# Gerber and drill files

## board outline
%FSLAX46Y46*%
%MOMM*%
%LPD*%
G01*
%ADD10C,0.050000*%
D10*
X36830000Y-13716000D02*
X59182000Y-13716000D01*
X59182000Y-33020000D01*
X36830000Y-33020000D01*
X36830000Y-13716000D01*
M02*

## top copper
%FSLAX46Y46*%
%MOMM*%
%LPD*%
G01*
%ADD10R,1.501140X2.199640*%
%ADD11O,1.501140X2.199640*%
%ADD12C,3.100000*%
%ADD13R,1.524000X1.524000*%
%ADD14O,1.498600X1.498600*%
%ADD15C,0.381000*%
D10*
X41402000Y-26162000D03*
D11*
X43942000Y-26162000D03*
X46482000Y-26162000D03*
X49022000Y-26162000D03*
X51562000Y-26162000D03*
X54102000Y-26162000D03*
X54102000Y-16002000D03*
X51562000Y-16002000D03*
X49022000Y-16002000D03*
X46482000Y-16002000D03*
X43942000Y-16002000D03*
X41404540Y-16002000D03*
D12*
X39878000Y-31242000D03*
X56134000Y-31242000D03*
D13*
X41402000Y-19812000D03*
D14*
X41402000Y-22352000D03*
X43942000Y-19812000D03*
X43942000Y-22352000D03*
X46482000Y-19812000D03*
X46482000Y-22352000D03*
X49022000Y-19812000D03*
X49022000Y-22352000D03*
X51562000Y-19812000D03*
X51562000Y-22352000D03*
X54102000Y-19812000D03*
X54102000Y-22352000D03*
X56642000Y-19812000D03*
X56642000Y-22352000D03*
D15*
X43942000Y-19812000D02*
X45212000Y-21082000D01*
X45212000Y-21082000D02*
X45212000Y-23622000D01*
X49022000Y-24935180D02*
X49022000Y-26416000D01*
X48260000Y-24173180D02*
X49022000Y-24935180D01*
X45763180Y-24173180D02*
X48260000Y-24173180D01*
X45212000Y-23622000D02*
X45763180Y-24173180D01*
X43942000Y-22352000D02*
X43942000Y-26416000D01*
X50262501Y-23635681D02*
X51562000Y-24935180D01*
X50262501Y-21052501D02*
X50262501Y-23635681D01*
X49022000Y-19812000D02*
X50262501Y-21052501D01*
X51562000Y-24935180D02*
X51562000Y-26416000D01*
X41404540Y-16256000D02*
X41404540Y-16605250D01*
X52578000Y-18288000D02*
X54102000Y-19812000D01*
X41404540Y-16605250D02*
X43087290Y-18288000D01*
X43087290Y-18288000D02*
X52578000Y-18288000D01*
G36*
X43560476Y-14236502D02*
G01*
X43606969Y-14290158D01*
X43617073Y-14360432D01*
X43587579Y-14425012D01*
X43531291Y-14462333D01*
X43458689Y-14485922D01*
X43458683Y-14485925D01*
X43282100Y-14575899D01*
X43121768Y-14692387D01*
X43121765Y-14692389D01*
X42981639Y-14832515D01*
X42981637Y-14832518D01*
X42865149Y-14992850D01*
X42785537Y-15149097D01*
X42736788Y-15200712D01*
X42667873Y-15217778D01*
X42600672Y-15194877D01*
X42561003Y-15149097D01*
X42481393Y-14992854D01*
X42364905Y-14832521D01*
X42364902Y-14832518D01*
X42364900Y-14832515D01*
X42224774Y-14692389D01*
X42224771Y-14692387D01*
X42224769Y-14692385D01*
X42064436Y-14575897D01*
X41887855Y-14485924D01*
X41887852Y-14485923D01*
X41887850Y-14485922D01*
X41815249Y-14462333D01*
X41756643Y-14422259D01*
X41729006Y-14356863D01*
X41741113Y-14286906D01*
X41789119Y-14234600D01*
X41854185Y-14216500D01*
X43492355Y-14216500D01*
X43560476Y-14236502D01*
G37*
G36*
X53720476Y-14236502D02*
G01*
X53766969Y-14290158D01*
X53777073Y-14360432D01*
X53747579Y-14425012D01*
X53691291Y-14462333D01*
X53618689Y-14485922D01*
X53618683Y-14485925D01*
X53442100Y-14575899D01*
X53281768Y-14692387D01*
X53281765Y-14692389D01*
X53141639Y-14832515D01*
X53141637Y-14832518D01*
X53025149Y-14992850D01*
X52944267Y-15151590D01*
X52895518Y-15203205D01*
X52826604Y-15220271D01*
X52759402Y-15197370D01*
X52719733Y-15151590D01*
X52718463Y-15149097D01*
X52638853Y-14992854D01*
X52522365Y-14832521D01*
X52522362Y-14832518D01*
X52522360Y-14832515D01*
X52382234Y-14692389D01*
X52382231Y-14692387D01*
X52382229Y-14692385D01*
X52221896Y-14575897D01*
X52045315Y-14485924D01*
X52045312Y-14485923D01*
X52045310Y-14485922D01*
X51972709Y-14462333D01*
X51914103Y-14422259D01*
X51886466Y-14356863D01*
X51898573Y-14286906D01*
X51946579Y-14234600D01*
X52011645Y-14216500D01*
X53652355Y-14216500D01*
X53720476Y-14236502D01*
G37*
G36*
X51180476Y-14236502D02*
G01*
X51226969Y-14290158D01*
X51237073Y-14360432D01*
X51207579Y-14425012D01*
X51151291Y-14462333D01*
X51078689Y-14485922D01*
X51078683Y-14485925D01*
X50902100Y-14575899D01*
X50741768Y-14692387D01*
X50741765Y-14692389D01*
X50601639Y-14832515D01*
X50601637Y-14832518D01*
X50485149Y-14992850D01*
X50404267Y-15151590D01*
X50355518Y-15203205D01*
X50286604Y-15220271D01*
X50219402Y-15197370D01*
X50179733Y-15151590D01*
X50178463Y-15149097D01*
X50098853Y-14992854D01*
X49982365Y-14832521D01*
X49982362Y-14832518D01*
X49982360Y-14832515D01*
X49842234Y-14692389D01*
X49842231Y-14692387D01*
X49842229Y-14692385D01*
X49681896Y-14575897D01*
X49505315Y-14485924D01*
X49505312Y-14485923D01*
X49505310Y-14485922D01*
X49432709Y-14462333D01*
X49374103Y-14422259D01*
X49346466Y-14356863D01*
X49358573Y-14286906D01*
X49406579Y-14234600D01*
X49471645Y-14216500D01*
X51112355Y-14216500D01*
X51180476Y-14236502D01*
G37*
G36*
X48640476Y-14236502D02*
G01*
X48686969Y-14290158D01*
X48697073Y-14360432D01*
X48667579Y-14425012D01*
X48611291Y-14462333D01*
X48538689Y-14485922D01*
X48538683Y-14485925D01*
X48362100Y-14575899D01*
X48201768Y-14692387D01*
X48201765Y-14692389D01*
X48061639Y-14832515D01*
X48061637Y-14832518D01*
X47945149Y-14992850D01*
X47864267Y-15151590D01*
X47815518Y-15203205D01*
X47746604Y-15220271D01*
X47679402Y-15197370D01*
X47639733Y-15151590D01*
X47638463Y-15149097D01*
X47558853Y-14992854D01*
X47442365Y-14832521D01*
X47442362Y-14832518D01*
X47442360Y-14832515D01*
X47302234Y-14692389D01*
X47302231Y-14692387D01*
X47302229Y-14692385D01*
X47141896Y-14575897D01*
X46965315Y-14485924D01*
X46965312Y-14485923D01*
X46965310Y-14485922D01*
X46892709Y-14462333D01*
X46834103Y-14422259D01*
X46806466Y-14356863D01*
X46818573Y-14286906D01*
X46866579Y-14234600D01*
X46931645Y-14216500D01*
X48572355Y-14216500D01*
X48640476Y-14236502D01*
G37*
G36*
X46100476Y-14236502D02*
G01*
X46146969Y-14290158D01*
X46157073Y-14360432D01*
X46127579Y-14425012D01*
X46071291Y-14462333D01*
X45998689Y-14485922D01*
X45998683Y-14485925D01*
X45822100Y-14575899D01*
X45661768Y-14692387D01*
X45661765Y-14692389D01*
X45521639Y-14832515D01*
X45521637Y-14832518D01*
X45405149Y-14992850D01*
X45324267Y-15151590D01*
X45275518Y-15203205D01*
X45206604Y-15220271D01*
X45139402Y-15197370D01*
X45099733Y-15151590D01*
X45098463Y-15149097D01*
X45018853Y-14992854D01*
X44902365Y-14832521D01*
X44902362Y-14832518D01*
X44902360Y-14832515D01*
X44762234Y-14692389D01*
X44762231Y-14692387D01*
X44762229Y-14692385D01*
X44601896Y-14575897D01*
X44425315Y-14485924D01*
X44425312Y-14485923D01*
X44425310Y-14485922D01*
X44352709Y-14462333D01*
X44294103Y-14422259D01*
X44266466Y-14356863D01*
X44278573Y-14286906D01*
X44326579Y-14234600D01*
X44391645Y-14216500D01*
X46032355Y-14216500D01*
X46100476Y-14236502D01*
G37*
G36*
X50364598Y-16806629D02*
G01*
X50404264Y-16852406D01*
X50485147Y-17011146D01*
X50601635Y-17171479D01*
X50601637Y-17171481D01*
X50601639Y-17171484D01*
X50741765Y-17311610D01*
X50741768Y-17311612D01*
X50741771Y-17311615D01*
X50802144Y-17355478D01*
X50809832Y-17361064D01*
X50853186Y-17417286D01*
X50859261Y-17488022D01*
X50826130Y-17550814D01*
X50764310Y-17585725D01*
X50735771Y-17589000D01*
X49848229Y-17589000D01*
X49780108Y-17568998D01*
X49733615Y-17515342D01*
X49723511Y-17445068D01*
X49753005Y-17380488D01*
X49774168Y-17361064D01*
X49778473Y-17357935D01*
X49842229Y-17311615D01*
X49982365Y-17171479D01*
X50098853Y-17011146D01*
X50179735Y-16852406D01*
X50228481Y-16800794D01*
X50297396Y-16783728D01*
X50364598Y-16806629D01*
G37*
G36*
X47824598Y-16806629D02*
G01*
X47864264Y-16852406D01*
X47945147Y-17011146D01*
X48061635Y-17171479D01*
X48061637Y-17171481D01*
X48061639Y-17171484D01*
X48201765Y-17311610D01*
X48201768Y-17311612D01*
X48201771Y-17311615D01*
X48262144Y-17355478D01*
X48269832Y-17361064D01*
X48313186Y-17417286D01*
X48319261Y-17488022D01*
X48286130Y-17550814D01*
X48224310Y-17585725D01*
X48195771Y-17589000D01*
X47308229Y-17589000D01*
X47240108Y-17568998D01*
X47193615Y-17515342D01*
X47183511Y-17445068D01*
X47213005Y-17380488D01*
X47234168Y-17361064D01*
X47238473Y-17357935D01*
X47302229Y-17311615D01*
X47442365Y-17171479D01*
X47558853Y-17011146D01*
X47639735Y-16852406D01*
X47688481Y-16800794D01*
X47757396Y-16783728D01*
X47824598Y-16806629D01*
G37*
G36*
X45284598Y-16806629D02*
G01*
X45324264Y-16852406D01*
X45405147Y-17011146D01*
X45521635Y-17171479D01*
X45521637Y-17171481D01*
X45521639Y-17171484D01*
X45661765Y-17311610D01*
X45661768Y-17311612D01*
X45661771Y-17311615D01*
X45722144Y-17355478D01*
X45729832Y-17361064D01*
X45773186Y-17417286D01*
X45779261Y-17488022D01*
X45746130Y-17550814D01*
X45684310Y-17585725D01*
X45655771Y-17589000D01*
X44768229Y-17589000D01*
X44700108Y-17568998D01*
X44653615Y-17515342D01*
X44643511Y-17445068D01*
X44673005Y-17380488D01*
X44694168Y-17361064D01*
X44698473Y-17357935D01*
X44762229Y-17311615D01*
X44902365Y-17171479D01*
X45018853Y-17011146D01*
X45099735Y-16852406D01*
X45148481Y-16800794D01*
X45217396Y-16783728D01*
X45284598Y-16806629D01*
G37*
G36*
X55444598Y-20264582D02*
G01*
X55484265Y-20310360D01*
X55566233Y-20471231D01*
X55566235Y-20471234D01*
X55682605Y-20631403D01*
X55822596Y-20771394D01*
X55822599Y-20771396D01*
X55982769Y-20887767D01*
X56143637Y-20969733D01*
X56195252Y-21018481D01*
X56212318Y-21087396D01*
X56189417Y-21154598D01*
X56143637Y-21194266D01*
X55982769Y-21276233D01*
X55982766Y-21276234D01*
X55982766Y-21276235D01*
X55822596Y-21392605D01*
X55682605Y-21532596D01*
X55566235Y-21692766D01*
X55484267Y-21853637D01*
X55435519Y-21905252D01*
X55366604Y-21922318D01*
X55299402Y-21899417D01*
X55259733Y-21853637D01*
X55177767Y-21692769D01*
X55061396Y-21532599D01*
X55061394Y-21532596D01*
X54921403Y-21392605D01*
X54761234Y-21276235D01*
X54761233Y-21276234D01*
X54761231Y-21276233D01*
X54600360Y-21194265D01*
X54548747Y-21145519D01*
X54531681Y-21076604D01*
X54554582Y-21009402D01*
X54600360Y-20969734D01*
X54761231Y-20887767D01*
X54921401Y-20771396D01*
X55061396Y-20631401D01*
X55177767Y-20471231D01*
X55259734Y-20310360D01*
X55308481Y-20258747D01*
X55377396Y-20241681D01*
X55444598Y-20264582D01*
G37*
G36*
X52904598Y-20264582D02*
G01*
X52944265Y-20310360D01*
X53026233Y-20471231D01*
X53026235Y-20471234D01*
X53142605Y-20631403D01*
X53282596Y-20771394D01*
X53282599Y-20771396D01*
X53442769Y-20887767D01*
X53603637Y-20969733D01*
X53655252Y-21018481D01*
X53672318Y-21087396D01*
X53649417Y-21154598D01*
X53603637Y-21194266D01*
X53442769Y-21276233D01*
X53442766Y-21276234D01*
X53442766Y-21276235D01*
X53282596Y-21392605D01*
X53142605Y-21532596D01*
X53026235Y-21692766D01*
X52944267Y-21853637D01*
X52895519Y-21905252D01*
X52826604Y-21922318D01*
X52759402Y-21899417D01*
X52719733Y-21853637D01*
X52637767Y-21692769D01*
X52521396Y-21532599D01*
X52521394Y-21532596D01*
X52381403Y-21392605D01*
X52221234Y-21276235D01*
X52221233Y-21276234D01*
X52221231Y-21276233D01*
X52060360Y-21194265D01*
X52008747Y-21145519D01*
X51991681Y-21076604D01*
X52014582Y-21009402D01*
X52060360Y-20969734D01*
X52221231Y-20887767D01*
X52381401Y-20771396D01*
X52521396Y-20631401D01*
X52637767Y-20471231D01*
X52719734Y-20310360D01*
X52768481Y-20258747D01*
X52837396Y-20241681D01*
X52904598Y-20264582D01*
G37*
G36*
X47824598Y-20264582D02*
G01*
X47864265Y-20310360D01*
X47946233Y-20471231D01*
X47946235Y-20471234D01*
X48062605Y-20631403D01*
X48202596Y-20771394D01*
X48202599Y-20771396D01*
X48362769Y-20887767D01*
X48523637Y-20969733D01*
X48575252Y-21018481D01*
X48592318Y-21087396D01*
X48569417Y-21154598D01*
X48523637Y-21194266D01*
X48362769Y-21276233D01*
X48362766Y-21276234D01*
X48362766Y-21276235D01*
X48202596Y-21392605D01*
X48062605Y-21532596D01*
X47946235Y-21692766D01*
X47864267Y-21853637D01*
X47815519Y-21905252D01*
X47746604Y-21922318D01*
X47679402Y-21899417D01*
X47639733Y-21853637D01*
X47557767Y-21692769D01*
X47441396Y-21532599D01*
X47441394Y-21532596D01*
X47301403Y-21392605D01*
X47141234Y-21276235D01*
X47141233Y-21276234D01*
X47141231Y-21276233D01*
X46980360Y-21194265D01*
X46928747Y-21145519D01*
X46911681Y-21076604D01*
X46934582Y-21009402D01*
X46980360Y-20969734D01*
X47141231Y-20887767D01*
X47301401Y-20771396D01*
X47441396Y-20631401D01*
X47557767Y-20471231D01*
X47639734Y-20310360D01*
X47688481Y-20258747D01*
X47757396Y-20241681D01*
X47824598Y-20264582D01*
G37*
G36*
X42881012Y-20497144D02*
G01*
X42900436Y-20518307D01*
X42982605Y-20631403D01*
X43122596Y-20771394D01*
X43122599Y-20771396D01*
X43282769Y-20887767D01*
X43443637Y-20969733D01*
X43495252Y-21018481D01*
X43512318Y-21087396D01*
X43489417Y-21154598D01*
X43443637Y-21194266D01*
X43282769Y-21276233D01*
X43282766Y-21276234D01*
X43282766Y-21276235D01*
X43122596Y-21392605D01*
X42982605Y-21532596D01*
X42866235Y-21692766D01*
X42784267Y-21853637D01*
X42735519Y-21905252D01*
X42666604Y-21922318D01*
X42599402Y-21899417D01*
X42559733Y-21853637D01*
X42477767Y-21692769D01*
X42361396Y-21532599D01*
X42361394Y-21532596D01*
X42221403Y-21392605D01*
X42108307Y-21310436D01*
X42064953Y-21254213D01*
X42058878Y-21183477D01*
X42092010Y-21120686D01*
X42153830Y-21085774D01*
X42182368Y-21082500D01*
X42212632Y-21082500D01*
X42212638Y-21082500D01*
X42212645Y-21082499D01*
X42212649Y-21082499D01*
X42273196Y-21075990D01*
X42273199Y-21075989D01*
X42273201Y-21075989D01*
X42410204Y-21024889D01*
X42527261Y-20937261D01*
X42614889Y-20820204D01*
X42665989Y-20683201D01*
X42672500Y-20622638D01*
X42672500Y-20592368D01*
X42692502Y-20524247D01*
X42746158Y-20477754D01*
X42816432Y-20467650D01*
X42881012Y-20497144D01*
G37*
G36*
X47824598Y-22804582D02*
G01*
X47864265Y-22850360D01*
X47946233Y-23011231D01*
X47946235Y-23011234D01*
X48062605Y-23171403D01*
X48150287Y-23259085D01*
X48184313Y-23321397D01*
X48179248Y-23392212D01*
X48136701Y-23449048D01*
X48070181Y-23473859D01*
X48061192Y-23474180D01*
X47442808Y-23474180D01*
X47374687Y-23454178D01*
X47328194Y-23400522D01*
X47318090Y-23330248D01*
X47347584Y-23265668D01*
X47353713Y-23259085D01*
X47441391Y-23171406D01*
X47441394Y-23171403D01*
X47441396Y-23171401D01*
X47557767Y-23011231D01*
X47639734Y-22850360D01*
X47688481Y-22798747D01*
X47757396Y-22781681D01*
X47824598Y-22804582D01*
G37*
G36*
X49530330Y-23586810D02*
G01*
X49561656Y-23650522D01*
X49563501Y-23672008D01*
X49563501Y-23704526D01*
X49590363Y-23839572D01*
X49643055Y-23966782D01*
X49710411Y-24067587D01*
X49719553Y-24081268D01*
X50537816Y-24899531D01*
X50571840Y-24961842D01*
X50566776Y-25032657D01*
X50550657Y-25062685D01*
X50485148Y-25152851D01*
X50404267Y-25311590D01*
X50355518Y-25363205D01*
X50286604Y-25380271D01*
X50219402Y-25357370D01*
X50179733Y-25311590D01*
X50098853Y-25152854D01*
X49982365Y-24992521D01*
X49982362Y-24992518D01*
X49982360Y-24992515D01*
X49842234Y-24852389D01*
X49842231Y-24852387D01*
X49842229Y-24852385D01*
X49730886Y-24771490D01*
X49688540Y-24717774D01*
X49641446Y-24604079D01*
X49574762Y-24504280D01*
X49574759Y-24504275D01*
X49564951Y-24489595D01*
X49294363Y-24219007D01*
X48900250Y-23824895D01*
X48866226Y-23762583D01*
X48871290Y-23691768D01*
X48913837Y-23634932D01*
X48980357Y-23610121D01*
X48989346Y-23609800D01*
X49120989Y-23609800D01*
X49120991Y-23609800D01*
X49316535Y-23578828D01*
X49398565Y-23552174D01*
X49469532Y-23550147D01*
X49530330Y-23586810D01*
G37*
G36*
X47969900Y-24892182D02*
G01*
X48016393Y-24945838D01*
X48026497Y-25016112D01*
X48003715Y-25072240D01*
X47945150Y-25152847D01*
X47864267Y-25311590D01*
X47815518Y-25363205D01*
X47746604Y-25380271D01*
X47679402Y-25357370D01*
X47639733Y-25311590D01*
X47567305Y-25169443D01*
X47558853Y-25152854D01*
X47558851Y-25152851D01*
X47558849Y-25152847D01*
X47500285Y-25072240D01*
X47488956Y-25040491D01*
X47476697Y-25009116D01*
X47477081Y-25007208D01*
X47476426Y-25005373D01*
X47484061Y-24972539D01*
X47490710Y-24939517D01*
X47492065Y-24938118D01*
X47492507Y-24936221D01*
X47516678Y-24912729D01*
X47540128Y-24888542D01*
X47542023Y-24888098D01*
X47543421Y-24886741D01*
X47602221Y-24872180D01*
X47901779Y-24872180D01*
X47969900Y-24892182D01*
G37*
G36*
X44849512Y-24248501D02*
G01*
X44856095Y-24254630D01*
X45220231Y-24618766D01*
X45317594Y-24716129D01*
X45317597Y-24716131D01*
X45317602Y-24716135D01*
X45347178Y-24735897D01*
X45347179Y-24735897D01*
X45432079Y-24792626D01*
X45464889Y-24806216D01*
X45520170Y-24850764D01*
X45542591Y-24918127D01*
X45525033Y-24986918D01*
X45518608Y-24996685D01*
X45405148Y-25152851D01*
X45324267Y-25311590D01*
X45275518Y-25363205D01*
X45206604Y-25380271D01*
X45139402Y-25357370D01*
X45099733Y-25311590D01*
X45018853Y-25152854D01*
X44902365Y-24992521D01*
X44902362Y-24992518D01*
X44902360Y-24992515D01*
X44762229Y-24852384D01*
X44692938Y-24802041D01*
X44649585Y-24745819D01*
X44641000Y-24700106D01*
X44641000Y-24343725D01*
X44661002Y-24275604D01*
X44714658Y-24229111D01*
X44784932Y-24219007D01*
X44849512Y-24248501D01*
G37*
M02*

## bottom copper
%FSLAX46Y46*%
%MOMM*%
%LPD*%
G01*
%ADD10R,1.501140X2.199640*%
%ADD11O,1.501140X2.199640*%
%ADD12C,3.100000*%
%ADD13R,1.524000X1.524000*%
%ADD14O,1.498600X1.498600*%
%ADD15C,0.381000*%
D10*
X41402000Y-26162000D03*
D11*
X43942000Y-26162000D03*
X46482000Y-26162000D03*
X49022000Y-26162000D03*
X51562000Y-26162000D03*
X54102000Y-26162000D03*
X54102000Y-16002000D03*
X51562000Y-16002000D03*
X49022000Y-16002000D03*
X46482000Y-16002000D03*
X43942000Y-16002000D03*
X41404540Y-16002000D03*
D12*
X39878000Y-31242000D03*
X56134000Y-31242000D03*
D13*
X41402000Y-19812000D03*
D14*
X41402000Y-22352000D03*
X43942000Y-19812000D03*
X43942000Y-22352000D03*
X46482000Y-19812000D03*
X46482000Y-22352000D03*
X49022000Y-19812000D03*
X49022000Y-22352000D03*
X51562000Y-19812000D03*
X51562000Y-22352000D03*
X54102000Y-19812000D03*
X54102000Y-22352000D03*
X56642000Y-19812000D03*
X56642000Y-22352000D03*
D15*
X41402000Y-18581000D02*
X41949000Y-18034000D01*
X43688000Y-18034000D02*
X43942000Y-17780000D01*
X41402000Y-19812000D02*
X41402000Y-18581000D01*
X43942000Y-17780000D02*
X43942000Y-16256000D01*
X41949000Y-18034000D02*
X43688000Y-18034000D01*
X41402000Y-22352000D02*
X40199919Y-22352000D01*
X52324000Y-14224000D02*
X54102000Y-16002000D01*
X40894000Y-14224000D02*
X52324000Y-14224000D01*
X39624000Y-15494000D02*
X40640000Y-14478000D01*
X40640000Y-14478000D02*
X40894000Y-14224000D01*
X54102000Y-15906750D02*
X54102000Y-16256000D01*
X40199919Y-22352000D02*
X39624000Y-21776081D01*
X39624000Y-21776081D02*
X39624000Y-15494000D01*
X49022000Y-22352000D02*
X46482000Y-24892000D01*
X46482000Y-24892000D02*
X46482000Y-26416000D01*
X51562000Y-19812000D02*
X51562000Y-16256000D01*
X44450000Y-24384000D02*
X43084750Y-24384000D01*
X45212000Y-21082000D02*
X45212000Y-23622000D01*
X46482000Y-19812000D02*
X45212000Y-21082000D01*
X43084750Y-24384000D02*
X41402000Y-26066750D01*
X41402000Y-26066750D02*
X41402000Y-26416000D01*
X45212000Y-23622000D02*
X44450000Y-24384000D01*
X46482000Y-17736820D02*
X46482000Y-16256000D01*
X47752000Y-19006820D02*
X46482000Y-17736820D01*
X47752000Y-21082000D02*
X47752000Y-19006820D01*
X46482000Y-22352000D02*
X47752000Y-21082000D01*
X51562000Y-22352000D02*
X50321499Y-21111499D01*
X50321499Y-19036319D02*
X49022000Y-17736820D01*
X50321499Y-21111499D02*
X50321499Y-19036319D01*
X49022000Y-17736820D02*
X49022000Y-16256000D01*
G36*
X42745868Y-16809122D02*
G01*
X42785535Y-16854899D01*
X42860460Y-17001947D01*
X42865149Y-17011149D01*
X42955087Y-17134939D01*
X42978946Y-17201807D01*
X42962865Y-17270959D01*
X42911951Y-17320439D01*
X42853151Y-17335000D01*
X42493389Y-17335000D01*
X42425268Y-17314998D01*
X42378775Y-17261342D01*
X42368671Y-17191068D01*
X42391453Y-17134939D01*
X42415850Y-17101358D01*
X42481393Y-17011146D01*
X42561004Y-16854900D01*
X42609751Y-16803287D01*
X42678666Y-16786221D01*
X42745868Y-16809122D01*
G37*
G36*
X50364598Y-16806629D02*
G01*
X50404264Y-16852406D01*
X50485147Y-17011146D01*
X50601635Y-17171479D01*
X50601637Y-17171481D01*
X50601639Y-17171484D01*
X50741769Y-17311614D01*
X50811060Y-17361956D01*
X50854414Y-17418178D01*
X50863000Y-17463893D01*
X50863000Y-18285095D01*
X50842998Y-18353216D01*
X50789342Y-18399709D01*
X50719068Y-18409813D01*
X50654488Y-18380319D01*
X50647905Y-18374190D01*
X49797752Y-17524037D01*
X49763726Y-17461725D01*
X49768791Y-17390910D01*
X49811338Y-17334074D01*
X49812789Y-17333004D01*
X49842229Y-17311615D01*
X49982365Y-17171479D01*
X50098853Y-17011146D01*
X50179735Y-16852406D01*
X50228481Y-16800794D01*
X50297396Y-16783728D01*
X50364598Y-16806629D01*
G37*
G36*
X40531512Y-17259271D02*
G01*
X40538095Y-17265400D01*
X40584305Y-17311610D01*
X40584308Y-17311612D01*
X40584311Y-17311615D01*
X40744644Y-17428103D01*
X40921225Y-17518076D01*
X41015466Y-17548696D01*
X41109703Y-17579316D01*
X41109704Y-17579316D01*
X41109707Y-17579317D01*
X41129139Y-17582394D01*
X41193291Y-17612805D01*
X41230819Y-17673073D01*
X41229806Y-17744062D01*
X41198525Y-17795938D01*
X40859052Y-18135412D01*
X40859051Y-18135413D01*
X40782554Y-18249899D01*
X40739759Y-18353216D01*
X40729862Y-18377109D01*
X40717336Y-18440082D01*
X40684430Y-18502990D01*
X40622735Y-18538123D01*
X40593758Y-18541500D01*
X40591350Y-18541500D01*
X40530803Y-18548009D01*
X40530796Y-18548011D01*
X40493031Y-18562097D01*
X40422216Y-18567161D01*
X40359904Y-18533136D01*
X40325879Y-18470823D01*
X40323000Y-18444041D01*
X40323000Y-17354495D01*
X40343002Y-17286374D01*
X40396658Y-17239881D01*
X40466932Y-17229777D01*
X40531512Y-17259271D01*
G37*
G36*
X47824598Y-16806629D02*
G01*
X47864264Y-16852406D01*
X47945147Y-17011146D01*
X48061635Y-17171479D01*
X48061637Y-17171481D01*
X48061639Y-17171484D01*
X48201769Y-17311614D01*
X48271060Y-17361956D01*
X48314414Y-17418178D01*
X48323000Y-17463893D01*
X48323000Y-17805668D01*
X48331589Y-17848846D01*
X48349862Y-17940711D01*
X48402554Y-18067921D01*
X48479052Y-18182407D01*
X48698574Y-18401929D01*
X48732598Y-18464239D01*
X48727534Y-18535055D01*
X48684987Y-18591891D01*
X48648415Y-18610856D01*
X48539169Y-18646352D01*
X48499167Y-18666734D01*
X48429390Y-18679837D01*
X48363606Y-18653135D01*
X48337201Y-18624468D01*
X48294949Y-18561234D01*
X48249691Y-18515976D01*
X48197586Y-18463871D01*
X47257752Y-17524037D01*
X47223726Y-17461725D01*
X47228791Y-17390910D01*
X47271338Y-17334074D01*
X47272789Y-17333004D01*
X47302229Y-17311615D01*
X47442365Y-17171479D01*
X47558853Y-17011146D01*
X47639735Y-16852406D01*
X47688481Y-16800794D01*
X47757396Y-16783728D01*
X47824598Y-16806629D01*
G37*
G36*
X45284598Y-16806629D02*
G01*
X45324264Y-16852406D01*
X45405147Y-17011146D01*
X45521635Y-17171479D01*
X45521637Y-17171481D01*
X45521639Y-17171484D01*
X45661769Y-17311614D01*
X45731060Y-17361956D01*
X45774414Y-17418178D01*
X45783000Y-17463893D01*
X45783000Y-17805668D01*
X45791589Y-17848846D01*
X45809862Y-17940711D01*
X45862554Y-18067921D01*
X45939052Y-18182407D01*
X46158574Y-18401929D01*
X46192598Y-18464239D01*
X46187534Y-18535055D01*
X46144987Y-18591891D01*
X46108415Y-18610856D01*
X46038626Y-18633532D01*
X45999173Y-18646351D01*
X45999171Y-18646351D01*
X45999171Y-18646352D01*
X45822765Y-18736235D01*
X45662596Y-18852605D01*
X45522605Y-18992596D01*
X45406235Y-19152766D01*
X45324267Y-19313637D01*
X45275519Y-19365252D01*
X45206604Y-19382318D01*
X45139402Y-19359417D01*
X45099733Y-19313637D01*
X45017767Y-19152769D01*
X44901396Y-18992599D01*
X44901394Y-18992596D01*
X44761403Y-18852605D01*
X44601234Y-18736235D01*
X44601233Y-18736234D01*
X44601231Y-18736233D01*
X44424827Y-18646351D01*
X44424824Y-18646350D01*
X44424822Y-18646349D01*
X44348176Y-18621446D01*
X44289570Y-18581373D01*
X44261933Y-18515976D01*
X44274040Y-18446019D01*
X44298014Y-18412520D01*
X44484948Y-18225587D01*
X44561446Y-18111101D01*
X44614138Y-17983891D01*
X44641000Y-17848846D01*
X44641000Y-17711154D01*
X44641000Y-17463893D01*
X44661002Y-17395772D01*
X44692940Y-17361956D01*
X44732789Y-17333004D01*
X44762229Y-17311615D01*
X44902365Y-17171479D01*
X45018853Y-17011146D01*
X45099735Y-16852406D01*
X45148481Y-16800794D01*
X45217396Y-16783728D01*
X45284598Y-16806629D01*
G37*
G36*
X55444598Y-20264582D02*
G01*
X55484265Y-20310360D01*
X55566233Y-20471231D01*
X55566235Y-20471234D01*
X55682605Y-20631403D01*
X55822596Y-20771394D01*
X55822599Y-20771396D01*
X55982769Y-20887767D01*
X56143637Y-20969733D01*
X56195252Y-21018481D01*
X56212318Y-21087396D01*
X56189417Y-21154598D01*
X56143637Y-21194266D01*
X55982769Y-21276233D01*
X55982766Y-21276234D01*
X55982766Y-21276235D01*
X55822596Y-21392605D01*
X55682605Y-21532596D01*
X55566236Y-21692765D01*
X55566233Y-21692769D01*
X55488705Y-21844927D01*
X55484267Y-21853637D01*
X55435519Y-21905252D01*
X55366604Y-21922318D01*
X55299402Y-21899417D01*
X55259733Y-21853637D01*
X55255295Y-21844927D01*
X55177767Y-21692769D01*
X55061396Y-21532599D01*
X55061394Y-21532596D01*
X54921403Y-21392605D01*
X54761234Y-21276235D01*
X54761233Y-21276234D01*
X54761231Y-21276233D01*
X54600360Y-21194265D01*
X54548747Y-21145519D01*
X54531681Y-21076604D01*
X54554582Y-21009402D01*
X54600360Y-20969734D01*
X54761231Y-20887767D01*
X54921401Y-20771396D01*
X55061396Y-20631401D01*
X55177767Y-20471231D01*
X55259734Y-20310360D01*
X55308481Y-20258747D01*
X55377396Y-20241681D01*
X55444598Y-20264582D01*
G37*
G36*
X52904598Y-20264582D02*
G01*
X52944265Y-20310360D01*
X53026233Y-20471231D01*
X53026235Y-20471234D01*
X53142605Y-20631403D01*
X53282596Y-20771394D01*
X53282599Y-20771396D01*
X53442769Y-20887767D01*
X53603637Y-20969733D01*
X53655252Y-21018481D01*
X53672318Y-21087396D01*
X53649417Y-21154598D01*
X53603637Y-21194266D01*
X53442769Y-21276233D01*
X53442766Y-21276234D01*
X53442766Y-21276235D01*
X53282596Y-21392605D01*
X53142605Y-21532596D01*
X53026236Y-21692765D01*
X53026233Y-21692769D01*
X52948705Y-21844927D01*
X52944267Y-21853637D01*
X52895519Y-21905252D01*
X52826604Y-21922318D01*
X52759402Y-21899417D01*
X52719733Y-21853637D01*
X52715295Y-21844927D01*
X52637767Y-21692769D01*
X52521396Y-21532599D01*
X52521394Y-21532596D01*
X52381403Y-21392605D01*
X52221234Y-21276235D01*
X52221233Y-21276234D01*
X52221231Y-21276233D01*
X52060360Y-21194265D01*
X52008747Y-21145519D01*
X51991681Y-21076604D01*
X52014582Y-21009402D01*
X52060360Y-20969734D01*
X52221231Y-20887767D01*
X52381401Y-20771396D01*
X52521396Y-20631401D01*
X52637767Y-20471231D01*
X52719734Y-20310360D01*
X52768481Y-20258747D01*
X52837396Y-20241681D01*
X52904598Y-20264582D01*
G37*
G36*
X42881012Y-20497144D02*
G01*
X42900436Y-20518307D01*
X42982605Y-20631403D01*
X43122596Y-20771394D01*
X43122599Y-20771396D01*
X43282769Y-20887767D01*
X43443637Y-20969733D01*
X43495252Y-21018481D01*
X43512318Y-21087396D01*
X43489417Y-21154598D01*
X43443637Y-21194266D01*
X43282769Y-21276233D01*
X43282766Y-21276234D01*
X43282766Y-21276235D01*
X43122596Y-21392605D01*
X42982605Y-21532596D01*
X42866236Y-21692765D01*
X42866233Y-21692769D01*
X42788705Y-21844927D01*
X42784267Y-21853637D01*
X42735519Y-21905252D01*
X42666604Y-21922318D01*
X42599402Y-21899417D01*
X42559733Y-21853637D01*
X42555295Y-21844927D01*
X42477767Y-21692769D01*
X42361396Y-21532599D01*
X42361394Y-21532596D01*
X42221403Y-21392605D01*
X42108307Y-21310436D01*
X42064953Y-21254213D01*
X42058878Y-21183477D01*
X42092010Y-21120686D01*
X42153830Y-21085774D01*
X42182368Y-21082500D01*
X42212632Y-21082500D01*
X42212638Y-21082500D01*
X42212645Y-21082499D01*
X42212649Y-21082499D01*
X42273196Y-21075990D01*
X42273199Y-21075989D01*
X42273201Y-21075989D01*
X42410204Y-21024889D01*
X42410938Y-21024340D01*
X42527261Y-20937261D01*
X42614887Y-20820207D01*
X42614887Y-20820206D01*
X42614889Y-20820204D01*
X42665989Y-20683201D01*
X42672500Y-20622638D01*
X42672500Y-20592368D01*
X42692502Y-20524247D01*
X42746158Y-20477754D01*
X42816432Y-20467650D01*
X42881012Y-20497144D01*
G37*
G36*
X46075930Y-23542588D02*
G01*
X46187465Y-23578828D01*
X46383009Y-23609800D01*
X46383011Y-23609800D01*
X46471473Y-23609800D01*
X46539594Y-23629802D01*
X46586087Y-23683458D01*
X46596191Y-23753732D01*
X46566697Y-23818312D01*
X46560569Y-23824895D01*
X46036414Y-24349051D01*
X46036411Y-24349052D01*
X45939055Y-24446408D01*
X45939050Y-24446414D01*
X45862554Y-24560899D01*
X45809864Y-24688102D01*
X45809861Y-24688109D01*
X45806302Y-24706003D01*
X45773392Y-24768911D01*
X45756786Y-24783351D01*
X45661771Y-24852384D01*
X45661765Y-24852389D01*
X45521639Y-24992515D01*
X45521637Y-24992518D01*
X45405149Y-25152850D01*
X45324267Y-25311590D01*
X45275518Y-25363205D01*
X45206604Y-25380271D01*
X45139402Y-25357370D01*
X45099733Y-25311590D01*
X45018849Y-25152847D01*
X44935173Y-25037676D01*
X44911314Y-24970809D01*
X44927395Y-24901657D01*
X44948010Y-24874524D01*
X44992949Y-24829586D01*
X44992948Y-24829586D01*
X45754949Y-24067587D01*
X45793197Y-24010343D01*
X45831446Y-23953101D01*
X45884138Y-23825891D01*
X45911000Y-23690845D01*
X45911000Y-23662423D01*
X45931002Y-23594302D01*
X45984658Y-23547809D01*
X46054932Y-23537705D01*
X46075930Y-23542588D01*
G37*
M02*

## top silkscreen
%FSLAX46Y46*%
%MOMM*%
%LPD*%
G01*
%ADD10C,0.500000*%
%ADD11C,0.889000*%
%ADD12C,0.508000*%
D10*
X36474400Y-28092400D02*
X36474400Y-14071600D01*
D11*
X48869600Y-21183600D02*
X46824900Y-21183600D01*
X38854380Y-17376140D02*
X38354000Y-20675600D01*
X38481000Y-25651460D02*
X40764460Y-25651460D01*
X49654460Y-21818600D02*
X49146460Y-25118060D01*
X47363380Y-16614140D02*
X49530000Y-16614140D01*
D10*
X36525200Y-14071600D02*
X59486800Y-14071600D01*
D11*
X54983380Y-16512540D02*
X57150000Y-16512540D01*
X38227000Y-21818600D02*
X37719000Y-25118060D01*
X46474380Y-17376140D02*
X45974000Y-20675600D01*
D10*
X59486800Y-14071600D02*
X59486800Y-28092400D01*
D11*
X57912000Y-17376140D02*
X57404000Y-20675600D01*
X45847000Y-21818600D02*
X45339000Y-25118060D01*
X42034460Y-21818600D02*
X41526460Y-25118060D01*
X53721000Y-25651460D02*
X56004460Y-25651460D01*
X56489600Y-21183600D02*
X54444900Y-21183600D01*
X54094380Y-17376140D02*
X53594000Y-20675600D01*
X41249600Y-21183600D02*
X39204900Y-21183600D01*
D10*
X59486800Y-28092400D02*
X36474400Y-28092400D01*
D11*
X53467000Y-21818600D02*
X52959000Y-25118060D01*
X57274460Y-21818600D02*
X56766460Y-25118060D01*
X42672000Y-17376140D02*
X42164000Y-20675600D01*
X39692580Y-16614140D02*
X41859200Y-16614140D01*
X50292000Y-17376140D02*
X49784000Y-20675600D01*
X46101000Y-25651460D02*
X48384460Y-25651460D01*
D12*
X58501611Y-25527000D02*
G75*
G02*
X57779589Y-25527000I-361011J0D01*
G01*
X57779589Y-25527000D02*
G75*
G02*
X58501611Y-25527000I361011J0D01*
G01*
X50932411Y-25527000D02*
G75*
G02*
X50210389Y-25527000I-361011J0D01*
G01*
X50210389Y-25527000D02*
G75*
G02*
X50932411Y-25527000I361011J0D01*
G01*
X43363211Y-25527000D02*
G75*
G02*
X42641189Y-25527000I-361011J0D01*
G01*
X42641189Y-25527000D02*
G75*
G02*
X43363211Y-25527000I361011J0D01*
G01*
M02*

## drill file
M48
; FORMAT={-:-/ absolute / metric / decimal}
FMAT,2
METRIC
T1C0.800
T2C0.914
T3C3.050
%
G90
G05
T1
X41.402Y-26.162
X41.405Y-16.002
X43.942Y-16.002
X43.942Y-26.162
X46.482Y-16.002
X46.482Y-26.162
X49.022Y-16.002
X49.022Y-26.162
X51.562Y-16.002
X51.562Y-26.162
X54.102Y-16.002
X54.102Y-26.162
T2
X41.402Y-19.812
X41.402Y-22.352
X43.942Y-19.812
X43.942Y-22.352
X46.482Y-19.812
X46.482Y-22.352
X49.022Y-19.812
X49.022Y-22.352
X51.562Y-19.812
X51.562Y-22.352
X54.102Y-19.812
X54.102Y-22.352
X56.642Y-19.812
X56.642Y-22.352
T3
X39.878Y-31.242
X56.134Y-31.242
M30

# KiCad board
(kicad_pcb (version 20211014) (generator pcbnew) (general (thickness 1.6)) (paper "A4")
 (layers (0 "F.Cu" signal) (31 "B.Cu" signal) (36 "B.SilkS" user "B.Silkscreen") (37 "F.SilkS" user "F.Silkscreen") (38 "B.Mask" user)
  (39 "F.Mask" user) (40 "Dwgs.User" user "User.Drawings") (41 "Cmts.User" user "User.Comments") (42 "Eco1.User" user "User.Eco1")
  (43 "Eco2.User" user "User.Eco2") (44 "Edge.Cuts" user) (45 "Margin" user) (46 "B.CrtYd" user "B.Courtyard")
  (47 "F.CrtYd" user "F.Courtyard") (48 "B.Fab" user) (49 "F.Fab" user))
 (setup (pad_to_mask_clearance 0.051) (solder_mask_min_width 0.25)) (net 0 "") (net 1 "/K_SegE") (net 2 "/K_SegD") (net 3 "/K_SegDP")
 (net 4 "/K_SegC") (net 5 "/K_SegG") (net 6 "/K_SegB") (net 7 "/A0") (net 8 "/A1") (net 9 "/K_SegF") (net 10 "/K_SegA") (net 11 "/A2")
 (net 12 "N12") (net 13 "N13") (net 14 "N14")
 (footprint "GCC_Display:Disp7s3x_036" (layer "F.Cu") (at 47.752 21.082)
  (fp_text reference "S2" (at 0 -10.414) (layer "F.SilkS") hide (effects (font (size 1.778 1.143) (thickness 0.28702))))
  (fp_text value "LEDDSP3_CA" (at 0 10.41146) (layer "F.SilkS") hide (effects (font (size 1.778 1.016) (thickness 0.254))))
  (fp_line (start -11.2776 7.0104) (end -11.2776 -7.0104) (layer "F.SilkS") (width 0.5))
  (fp_line (start 1.1176 0.1016) (end -0.9271 0.1016) (layer "F.SilkS") (width 0.889))
  (fp_line (start -8.89762 -3.70586) (end -9.398 -0.4064) (layer "F.SilkS") (width 0.889))
  (fp_line (start -9.271 4.56946) (end -6.98754 4.56946) (layer "F.SilkS") (width 0.889))
  (fp_line (start 1.90246 0.7366) (end 1.39446 4.03606) (layer "F.SilkS") (width 0.889))
  (fp_line (start -0.38862 -4.46786) (end 1.778 -4.46786) (layer "F.SilkS") (width 0.889))
  (fp_line (start -11.2268 -7.0104) (end 11.7348 -7.0104) (layer "F.SilkS") (width 0.5))
  (fp_line (start 7.23138 -4.56946) (end 9.398 -4.56946) (layer "F.SilkS") (width 0.889))
  (fp_line (start -9.525 0.7366) (end -10.033 4.03606) (layer "F.SilkS") (width 0.889))
  (fp_line (start -1.27762 -3.70586) (end -1.778 -0.4064) (layer "F.SilkS") (width 0.889))
  (fp_line (start 11.7348 -7.0104) (end 11.7348 7.0104) (layer "F.SilkS") (width 0.5))
  (fp_line (start 10.16 -3.70586) (end 9.652 -0.4064) (layer "F.SilkS") (width 0.889))
  (fp_line (start -1.905 0.7366) (end -2.413 4.03606) (layer "F.SilkS") (width 0.889))
  (fp_line (start -5.71754 0.7366) (end -6.22554 4.03606) (layer "F.SilkS") (width 0.889))
  (fp_line (start 5.969 4.56946) (end 8.25246 4.56946) (layer "F.SilkS") (width 0.889))
  (fp_line (start 8.7376 0.1016) (end 6.6929 0.1016) (layer "F.SilkS") (width 0.889))
  (fp_line (start 6.34238 -3.70586) (end 5.842 -0.4064) (layer "F.SilkS") (width 0.889))
  (fp_line (start -6.5024 0.1016) (end -8.5471 0.1016) (layer "F.SilkS") (width 0.889))
  (fp_line (start 11.7348 7.0104) (end -11.2776 7.0104) (layer "F.SilkS") (width 0.5))
  (fp_line (start 5.715 0.7366) (end 5.207 4.03606) (layer "F.SilkS") (width 0.889))
  (fp_line (start 9.52246 0.7366) (end 9.01446 4.03606) (layer "F.SilkS") (width 0.889))
  (fp_line (start -5.08 -3.70586) (end -5.588 -0.4064) (layer "F.SilkS") (width 0.889))
  (fp_line (start -8.05942 -4.46786) (end -5.8928 -4.46786) (layer "F.SilkS") (width 0.889))
  (fp_line (start 2.54 -3.70586) (end 2.032 -0.4064) (layer "F.SilkS") (width 0.889))
  (fp_line (start -1.651 4.56946) (end 0.63246 4.56946) (layer "F.SilkS") (width 0.889))
  (fp_circle (center 10.3886 4.445) (end 10.6426 4.18846) (layer "F.SilkS") (width 0.508) (fill none))
  (fp_circle (center 2.8194 4.445) (end 3.0734 4.18846) (layer "F.SilkS") (width 0.508) (fill none))
  (fp_circle (center -4.7498 4.445) (end -4.4958 4.18846) (layer "F.SilkS") (width 0.508) (fill none))
  (pad "1" thru_hole rect locked (at -6.35 5.08 90) (size 2.19964 1.50114) (drill 0.8001) (layers *.Cu *.Mask) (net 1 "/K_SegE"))
  (pad "2" thru_hole oval locked (at -3.81 5.08 90) (size 2.19964 1.50114) (drill 0.8001) (layers *.Cu *.Mask) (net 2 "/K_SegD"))
  (pad "3" thru_hole oval locked (at -1.27 5.08 90) (size 2.19964 1.50114) (drill 0.8001) (layers *.Cu *.Mask) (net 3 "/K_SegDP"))
  (pad "4" thru_hole oval locked (at 1.27 5.08 90) (size 2.19964 1.50114) (drill 0.8001) (layers *.Cu *.Mask) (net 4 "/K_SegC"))
  (pad "5" thru_hole oval locked (at 3.81 5.08 90) (size 2.19964 1.50114) (drill 0.8001) (layers *.Cu *.Mask) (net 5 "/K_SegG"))
  (pad "6" thru_hole oval locked (at 6.35 5.08 90) (size 2.19964 1.50114) (drill 0.8001) (layers *.Cu *.Mask))
  (pad "7" thru_hole oval locked (at 6.35 -5.08 90) (size 2.19964 1.50114) (drill 0.8001) (layers *.Cu *.Mask) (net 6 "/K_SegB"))
  (pad "8" thru_hole oval locked (at 3.81 -5.08 90) (size 2.19964 1.50114) (drill 0.8001) (layers *.Cu *.Mask) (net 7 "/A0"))
  (pad "9" thru_hole oval locked (at 1.27 -5.08 90) (size 2.19964 1.50114) (drill 0.8001) (layers *.Cu *.Mask) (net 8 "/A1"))
  (pad "10" thru_hole oval locked (at -1.27 -5.08 90) (size 2.19964 1.50114) (drill 0.8001) (layers *.Cu *.Mask) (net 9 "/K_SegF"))
  (pad "11" thru_hole oval locked (at -3.81 -5.08 90) (size 2.19964 1.50114) (drill 0.8001) (layers *.Cu *.Mask) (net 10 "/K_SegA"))
  (pad "12" thru_hole oval locked (at -6.34746 -5.08 90) (size 2.19964 1.50114) (drill 0.8001) (layers *.Cu *.Mask) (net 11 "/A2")))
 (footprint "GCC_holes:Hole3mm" (layer "B.Cu") (at 39.878 31.242)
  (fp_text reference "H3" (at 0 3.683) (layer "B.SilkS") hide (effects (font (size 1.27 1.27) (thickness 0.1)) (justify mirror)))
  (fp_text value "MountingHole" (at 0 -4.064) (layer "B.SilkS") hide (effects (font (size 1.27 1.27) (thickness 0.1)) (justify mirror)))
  (pad "1" thru_hole circle locked (at 0 0) (size 3.1 3.1) (drill 3.05) (layers *.Cu *.Mask)))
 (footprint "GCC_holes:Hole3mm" (layer "B.Cu") (at 56.134 31.242)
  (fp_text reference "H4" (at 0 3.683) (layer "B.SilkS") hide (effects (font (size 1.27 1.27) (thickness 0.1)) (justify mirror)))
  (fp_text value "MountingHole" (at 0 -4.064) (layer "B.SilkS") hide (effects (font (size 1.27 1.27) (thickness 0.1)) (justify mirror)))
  (pad "1" thru_hole circle locked (at 0 0) (size 3.1 3.1) (drill 3.05) (layers *.Cu *.Mask)))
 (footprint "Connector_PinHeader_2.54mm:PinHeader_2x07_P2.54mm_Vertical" (layer "B.Cu") (at 41.402 19.812 -90)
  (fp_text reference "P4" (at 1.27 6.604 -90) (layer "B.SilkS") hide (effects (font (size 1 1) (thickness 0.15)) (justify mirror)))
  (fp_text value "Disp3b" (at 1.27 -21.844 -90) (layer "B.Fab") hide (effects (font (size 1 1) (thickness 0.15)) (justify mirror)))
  (pad "1" thru_hole rect locked (at 0 0 270) (size 1.524 1.524) (drill 0.9144) (layers *.Cu *.Mask) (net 10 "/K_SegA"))
  (pad "2" thru_hole oval locked (at 2.54 0 270) (size 1.4986 1.4986) (drill 0.9144) (layers *.Cu *.Mask) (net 6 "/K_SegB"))
  (pad "3" thru_hole oval locked (at 0 -2.54 270) (size 1.4986 1.4986) (drill 0.9144) (layers *.Cu *.Mask) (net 4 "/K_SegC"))
  (pad "4" thru_hole oval locked (at 2.54 -2.54 270) (size 1.4986 1.4986) (drill 0.9144) (layers *.Cu *.Mask) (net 2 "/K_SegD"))
  (pad "5" thru_hole oval locked (at 0 -5.08 270) (size 1.4986 1.4986) (drill 0.9144) (layers *.Cu *.Mask) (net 1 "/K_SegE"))
  (pad "6" thru_hole oval locked (at 2.54 -5.08 270) (size 1.4986 1.4986) (drill 0.9144) (layers *.Cu *.Mask) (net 9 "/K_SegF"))
  (pad "7" thru_hole oval locked (at 0 -7.62 270) (size 1.4986 1.4986) (drill 0.9144) (layers *.Cu *.Mask) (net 5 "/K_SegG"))
  (pad "8" thru_hole oval locked (at 2.54 -7.62 270) (size 1.4986 1.4986) (drill 0.9144) (layers *.Cu *.Mask) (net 3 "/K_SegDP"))
  (pad "9" thru_hole oval locked (at 0 -10.16 270) (size 1.4986 1.4986) (drill 0.9144) (layers *.Cu *.Mask) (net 7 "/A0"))
  (pad "10" thru_hole oval locked (at 2.54 -10.16 270) (size 1.4986 1.4986) (drill 0.9144) (layers *.Cu *.Mask) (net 8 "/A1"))
  (pad "11" thru_hole oval locked (at 0 -12.7 270) (size 1.4986 1.4986) (drill 0.9144) (layers *.Cu *.Mask) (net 11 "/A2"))
  (pad "12" thru_hole oval locked (at 2.54 -12.7 270) (size 1.4986 1.4986) (drill 0.9144) (layers *.Cu *.Mask) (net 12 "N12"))
  (pad "13" thru_hole oval locked (at 0 -15.24 270) (size 1.4986 1.4986) (drill 0.9144) (layers *.Cu *.Mask) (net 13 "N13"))
  (pad "14" thru_hole oval locked (at 2.54 -15.24 270) (size 1.4986 1.4986) (drill 0.9144) (layers *.Cu *.Mask) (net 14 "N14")))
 (gr_rect (start 36.83 13.716) (end 59.182 33.02) (layer "Edge.Cuts") (width 0.05) (fill none))
 (segment (start 41.402 18.581) (end 41.949 18.034) (width 0.381) (layer "B.Cu") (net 10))
 (segment (start 43.688 18.034) (end 43.942 17.78) (width 0.381) (layer "B.Cu") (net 10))
 (segment (start 41.402 19.812) (end 41.402 18.581) (width 0.381) (layer "B.Cu") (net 10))
 (segment (start 43.942 17.78) (end 43.942 16.256) (width 0.381) (layer "B.Cu") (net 10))
 (segment (start 41.949 18.034) (end 43.688 18.034) (width 0.381) (layer "B.Cu") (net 10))
 (segment (start 41.402 22.352) (end 40.199919 22.352) (width 0.381) (layer "B.Cu") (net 6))
 (segment (start 52.324 14.224) (end 54.102 16.002) (width 0.381) (layer "B.Cu") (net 6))
 (segment (start 40.894 14.224) (end 52.324 14.224) (width 0.381) (layer "B.Cu") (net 6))
 (segment (start 39.624 15.494) (end 40.64 14.478) (width 0.381) (layer "B.Cu") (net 6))
 (segment (start 40.64 14.478) (end 40.894 14.224) (width 0.381) (layer "B.Cu") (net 6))
 (segment (start 54.102 15.90675) (end 54.102 16.256) (width 0.381) (layer "B.Cu") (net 6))
 (segment (start 40.199919 22.352) (end 39.624 21.776081) (width 0.381) (layer "B.Cu") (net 6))
 (segment (start 39.624 21.776081) (end 39.624 15.494) (width 0.381) (layer "B.Cu") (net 6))
 (segment (start 43.942 19.812) (end 45.212 21.082) (width 0.381) (layer "F.Cu") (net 4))
 (segment (start 45.212 21.082) (end 45.212 23.622) (width 0.381) (layer "F.Cu") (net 4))
 (segment (start 49.022 24.93518) (end 49.022 26.416) (width 0.381) (layer "F.Cu") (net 4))
 (segment (start 48.26 24.17318) (end 49.022 24.93518) (width 0.381) (layer "F.Cu") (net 4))
 (segment (start 45.76318 24.17318) (end 48.26 24.17318) (width 0.381) (layer "F.Cu") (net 4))
 (segment (start 45.212 23.622) (end 45.76318 24.17318) (width 0.381) (layer "F.Cu") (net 4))
 (segment (start 49.022 22.352) (end 46.482 24.892) (width 0.381) (layer "B.Cu") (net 3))
 (segment (start 46.482 24.892) (end 46.482 26.416) (width 0.381) (layer "B.Cu") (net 3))
 (segment (start 51.562 19.812) (end 51.562 16.256) (width 0.381) (layer "B.Cu") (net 7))
 (segment (start 43.942 22.352) (end 43.942 26.416) (width 0.381) (layer "F.Cu") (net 2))
 (segment (start 44.45 24.384) (end 43.08475 24.384) (width 0.381) (layer "B.Cu") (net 1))
 (segment (start 45.212 21.082) (end 45.212 23.622) (width 0.381) (layer "B.Cu") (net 1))
 (segment (start 46.482 19.812) (end 45.212 21.082) (width 0.381) (layer "B.Cu") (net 1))
 (segment (start 43.08475 24.384) (end 41.402 26.06675) (width 0.381) (layer "B.Cu") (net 1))
 (segment (start 41.402 26.06675) (end 41.402 26.416) (width 0.381) (layer "B.Cu") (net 1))
 (segment (start 45.212 23.622) (end 44.45 24.384) (width 0.381) (layer "B.Cu") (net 1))
 (segment (start 50.262501 23.635681) (end 51.562 24.93518) (width 0.381) (layer "F.Cu") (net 5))
 (segment (start 50.262501 21.052501) (end 50.262501 23.635681) (width 0.381) (layer "F.Cu") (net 5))
 (segment (start 49.022 19.812) (end 50.262501 21.052501) (width 0.381) (layer "F.Cu") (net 5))
 (segment (start 51.562 24.93518) (end 51.562 26.416) (width 0.381) (layer "F.Cu") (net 5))
 (segment (start 46.482 17.73682) (end 46.482 16.256) (width 0.381) (layer "B.Cu") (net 9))
 (segment (start 47.752 19.00682) (end 46.482 17.73682) (width 0.381) (layer "B.Cu") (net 9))
 (segment (start 47.752 21.082) (end 47.752 19.00682) (width 0.381) (layer "B.Cu") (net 9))
 (segment (start 46.482 22.352) (end 47.752 21.082) (width 0.381) (layer "B.Cu") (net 9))
 (segment (start 51.562 22.352) (end 50.321499 21.111499) (width 0.381) (layer "B.Cu") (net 8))
 (segment (start 50.321499 19.036319) (end 49.022 17.73682) (width 0.381) (layer "B.Cu") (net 8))
 (segment (start 50.321499 21.111499) (end 50.321499 19.036319) (width 0.381) (layer "B.Cu") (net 8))
 (segment (start 49.022 17.73682) (end 49.022 16.256) (width 0.381) (layer "B.Cu") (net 8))
 (segment (start 41.40454 16.256) (end 41.40454 16.60525) (width 0.381) (layer "F.Cu") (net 11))
 (segment (start 52.578 18.288) (end 54.102 19.812) (width 0.381) (layer "F.Cu") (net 11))
 (segment (start 41.40454 16.60525) (end 43.08729 18.288) (width 0.381) (layer "F.Cu") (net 11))
 (segment (start 43.08729 18.288) (end 52.578 18.288) (width 0.381) (layer "F.Cu") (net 11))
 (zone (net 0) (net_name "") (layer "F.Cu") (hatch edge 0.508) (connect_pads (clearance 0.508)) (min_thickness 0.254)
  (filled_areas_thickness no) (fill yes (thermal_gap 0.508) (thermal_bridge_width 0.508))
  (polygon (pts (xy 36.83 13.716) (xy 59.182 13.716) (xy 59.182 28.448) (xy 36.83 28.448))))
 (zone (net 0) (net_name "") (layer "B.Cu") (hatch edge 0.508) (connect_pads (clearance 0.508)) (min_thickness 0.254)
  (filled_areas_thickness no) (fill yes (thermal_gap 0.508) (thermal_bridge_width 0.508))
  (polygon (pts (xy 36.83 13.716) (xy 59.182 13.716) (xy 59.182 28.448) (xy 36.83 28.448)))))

